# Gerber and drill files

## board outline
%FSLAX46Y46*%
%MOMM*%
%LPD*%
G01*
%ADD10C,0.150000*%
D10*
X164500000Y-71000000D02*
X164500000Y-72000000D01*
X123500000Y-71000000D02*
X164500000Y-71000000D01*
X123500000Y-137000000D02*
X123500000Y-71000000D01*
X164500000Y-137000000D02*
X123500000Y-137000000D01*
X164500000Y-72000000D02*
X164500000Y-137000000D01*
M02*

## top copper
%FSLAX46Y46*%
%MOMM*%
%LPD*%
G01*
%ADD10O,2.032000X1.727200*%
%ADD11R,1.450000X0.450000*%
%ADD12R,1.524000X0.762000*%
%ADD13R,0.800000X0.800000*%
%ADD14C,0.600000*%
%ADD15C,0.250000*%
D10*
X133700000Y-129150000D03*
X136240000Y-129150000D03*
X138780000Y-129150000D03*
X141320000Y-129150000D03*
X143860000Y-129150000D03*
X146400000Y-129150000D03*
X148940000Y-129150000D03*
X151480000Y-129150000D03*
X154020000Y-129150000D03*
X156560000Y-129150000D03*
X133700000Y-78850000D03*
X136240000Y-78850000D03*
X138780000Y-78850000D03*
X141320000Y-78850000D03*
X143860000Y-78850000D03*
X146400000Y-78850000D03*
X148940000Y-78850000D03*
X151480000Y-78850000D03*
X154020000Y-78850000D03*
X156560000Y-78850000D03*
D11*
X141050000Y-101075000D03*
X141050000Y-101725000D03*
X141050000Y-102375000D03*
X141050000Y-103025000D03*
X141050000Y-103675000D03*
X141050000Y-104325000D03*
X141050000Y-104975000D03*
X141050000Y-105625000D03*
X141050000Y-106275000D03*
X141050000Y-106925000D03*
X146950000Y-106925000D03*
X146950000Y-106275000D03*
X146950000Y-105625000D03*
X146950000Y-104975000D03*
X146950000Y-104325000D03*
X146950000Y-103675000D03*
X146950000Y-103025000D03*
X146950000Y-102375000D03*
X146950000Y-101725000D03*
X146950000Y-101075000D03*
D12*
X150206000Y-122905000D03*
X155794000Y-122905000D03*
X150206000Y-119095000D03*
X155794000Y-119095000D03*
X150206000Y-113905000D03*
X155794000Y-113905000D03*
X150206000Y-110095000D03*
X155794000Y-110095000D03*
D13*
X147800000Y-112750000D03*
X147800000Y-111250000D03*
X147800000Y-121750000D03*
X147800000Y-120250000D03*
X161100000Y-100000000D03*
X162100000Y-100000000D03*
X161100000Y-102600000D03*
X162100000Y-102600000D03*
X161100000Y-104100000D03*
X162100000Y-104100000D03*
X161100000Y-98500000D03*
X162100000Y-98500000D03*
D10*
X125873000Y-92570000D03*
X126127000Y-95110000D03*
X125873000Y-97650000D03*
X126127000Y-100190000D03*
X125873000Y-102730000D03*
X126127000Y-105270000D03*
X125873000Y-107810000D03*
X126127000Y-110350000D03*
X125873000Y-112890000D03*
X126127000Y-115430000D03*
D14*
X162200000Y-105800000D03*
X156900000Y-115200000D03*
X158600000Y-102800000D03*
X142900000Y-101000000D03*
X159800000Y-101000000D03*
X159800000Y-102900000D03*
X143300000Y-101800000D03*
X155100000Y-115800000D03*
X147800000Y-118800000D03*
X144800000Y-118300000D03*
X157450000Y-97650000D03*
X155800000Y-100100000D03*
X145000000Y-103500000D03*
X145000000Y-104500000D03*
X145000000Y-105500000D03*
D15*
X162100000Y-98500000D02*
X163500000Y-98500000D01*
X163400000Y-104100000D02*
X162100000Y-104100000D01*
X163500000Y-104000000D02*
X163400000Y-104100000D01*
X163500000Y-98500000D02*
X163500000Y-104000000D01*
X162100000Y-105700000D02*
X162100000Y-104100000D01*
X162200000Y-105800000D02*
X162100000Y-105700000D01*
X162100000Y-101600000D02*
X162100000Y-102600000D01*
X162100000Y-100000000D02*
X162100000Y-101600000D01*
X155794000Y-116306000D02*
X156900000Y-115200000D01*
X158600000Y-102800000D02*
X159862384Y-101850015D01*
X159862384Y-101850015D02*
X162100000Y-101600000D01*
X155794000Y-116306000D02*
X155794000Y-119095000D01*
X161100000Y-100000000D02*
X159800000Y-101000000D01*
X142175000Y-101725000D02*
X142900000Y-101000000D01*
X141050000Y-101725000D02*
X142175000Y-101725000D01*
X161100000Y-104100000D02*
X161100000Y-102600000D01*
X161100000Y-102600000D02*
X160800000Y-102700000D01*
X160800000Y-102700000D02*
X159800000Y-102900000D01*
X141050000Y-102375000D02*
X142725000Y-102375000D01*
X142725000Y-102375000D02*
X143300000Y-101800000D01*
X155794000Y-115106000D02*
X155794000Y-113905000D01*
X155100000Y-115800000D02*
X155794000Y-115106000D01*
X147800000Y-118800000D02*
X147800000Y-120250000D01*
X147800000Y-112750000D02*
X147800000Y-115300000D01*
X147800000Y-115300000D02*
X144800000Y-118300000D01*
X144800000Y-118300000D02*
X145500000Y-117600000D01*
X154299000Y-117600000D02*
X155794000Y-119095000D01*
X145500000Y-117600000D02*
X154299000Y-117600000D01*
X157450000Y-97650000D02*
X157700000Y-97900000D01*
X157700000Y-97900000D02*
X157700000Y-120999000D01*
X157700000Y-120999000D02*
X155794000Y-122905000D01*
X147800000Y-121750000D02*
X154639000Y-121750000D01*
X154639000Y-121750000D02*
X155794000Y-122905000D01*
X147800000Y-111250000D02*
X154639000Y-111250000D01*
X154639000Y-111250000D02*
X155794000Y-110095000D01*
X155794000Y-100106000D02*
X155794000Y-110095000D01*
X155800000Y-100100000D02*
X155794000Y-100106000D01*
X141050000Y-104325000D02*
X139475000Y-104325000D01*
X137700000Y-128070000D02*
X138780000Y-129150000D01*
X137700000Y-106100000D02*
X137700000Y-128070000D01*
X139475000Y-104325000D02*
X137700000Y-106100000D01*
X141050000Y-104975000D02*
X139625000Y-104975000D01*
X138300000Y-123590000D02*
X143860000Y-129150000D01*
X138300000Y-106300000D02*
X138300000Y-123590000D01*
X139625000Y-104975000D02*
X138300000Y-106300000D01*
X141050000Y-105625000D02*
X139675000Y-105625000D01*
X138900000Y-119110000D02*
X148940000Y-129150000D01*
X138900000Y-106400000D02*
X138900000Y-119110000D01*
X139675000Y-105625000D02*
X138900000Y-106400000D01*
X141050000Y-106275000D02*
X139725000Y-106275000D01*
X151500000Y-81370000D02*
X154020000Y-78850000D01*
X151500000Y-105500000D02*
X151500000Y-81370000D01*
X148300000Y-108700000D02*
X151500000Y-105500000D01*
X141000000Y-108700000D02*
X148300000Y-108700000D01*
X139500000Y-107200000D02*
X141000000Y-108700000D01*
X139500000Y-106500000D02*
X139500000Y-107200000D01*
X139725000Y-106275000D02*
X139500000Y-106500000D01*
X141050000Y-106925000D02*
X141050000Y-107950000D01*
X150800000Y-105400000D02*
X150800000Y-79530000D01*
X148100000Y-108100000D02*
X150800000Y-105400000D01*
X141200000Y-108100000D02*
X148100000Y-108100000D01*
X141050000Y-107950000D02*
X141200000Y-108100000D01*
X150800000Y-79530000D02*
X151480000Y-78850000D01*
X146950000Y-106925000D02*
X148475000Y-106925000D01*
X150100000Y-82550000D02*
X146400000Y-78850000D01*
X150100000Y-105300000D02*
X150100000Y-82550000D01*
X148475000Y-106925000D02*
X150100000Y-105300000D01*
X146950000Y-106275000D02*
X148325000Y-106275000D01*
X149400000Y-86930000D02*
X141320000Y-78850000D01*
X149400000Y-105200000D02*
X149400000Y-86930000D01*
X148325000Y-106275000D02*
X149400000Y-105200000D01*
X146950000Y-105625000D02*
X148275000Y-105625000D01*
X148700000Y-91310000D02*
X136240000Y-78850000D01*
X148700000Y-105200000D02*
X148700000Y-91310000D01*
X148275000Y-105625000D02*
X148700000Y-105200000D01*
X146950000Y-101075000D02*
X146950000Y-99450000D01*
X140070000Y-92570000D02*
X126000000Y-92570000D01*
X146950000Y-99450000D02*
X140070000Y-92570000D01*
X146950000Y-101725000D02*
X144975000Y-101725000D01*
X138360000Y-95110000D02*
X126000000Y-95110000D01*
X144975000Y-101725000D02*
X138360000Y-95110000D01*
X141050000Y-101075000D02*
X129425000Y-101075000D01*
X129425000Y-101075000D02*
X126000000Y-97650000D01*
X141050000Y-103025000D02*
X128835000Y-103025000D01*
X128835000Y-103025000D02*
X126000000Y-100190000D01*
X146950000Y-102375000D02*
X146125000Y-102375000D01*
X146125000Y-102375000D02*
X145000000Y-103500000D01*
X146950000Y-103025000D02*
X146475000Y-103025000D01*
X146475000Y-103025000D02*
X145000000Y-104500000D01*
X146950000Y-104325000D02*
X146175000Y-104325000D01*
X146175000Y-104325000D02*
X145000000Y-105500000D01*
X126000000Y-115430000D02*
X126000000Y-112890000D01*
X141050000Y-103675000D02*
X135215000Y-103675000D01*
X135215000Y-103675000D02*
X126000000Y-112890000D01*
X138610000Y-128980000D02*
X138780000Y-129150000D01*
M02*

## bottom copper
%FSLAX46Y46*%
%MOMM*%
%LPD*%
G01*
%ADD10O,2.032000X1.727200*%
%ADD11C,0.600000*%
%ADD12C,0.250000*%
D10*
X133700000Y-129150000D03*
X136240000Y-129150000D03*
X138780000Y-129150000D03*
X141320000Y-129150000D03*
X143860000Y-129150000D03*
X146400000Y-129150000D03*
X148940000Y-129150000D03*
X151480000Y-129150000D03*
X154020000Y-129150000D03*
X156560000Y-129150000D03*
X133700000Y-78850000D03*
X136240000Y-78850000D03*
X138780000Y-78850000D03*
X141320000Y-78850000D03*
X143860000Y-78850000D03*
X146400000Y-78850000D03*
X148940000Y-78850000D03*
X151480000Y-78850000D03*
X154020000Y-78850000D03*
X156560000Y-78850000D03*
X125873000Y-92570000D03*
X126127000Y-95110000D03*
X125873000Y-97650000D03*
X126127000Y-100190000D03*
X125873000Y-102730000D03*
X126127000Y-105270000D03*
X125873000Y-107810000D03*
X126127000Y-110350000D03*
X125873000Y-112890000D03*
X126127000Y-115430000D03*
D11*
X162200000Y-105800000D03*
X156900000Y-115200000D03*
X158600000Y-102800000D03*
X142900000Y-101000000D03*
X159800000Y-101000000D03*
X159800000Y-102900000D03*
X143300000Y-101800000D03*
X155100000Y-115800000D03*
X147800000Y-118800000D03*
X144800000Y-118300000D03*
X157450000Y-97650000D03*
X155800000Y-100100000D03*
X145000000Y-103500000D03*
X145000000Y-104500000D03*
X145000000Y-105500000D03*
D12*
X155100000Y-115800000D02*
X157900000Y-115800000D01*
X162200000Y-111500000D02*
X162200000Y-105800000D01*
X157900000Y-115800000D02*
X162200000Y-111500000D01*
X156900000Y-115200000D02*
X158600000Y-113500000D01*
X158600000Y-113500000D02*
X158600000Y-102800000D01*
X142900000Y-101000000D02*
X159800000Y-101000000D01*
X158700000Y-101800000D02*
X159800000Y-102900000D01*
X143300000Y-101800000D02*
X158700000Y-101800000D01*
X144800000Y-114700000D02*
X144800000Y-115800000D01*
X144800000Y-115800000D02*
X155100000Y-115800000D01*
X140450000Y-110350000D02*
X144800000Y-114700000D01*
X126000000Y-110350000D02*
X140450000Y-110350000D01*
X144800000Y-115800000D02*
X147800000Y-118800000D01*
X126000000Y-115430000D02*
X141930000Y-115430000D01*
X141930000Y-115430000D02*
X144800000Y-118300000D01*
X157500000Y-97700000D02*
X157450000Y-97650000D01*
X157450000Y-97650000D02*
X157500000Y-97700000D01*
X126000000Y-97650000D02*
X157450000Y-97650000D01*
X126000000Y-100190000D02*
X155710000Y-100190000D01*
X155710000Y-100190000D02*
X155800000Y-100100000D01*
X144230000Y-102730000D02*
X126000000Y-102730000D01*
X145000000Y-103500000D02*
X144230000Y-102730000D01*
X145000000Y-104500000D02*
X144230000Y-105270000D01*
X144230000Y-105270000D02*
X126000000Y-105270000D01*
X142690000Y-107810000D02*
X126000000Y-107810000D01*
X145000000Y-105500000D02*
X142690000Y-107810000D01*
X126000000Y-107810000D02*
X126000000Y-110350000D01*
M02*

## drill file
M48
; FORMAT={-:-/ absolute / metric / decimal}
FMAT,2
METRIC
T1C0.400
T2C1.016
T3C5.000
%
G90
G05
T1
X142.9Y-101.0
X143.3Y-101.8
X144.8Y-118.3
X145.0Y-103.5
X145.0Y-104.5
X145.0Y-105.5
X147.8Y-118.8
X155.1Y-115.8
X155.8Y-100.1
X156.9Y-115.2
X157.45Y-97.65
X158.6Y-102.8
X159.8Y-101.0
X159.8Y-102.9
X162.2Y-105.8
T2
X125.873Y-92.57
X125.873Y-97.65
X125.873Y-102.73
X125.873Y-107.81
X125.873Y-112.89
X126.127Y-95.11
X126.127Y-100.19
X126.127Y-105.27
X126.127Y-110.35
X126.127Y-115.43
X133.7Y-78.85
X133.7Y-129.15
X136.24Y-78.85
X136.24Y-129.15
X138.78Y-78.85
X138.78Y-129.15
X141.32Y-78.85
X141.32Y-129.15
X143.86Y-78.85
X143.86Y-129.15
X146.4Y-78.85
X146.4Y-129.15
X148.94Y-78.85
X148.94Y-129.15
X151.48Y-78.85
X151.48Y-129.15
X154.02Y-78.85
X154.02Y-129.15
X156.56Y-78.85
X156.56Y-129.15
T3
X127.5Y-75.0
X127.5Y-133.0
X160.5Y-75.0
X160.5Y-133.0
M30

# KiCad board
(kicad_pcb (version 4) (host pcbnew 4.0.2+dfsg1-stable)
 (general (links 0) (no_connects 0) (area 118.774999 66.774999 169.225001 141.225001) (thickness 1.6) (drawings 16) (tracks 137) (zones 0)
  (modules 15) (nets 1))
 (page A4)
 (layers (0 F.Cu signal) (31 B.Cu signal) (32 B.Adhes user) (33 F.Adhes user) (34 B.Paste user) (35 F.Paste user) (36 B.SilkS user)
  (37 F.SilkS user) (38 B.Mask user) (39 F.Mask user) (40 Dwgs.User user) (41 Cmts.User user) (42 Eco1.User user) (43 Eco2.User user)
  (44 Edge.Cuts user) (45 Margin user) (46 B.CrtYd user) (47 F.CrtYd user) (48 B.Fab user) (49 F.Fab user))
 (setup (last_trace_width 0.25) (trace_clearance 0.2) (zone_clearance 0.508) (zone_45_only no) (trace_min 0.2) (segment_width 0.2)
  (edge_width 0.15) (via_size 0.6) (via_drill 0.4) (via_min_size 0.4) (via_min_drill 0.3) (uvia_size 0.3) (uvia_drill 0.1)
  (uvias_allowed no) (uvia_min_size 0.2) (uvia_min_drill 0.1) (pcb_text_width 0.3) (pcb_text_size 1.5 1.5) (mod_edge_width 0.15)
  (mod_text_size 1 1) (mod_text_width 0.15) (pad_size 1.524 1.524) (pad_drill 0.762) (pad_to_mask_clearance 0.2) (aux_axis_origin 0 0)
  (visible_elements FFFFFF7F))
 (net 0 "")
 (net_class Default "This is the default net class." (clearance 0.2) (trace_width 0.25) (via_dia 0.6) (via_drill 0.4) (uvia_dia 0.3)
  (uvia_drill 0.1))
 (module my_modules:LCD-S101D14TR (layer B.Cu) (at 144 104 180)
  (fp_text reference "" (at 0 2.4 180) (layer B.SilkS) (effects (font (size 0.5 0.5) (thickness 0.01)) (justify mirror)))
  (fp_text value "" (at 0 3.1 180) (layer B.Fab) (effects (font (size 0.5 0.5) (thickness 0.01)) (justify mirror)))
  (pad 10 thru_hole oval (at 10.3 -25.15 180) (size 2.032 1.7272) (drill 1.016) (layers *.Cu *.Mask B.SilkS))
  (pad 9 thru_hole oval (at 7.76 -25.15 180) (size 2.032 1.7272) (drill 1.016) (layers *.Cu *.Mask B.SilkS))
  (pad 8 thru_hole oval (at 5.22 -25.15 180) (size 2.032 1.7272) (drill 1.016) (layers *.Cu *.Mask B.SilkS))
  (pad 7 thru_hole oval (at 2.68 -25.15 180) (size 2.032 1.7272) (drill 1.016) (layers *.Cu *.Mask B.SilkS))
  (pad 6 thru_hole oval (at 0.14 -25.15 180) (size 2.032 1.7272) (drill 1.016) (layers *.Cu *.Mask B.SilkS))
  (pad 5 thru_hole oval (at -2.4 -25.15 180) (size 2.032 1.7272) (drill 1.016) (layers *.Cu *.Mask B.SilkS))
  (pad 4 thru_hole oval (at -4.94 -25.15 180) (size 2.032 1.7272) (drill 1.016) (layers *.Cu *.Mask B.SilkS))
  (pad 3 thru_hole oval (at -7.48 -25.15 180) (size 2.032 1.7272) (drill 1.016) (layers *.Cu *.Mask B.SilkS))
  (pad 2 thru_hole oval (at -10.02 -25.15 180) (size 2.032 1.7272) (drill 1.016) (layers *.Cu *.Mask B.SilkS))
  (pad 1 thru_hole oval (at -12.56 -25.15 180) (size 2.032 1.7272) (drill 1.016) (layers *.Cu *.Mask B.SilkS))
  (pad 11 thru_hole oval (at 10.3 25.15 180) (size 2.032 1.7272) (drill 1.016) (layers *.Cu *.Mask B.SilkS))
  (pad 12 thru_hole oval (at 7.76 25.15 180) (size 2.032 1.7272) (drill 1.016) (layers *.Cu *.Mask B.SilkS))
  (pad 13 thru_hole oval (at 5.22 25.15 180) (size 2.032 1.7272) (drill 1.016) (layers *.Cu *.Mask B.SilkS))
  (pad 14 thru_hole oval (at 2.68 25.15 180) (size 2.032 1.7272) (drill 1.016) (layers *.Cu *.Mask B.SilkS))
  (pad 15 thru_hole oval (at 0.14 25.15 180) (size 2.032 1.7272) (drill 1.016) (layers *.Cu *.Mask B.SilkS))
  (pad 16 thru_hole oval (at -2.4 25.15 180) (size 2.032 1.7272) (drill 1.016) (layers *.Cu *.Mask B.SilkS))
  (pad 17 thru_hole oval (at -4.94 25.15 180) (size 2.032 1.7272) (drill 1.016) (layers *.Cu *.Mask B.SilkS))
  (pad 18 thru_hole oval (at -7.48 25.15 180) (size 2.032 1.7272) (drill 1.016) (layers *.Cu *.Mask B.SilkS))
  (pad 19 thru_hole oval (at -10.02 25.15 180) (size 2.032 1.7272) (drill 1.016) (layers *.Cu *.Mask B.SilkS))
  (pad 20 thru_hole oval (at -12.56 25.15 180) (size 2.032 1.7272) (drill 1.016) (layers *.Cu *.Mask B.SilkS)))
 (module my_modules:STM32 (layer F.Cu) (at 144 104)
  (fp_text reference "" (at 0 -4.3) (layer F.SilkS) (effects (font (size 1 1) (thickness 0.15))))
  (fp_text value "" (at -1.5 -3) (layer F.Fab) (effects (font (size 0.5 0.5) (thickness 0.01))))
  (pad BOOT smd rect (at -2.95 -2.925) (size 1.45 0.45) (layers F.Cu F.Paste F.Mask))
  (pad 2 smd rect (at -2.95 -2.275) (size 1.45 0.45) (layers F.Cu F.Paste F.Mask))
  (pad 3 smd rect (at -2.95 -1.625) (size 1.45 0.45) (layers F.Cu F.Paste F.Mask))
  (pad NRST smd rect (at -2.95 -0.975) (size 1.45 0.45) (layers F.Cu F.Paste F.Mask))
  (pad VCC smd rect (at -2.95 -0.325) (size 1.45 0.45) (layers F.Cu F.Paste F.Mask))
  (pad PA0 smd rect (at -2.95 0.325) (size 1.45 0.45) (layers F.Cu F.Paste F.Mask))
  (pad PA1 smd rect (at -2.95 0.975) (size 1.45 0.45) (layers F.Cu F.Paste F.Mask))
  (pad PA2 smd rect (at -2.95 1.625) (size 1.45 0.45) (layers F.Cu F.Paste F.Mask))
  (pad PA3 smd rect (at -2.95 2.275) (size 1.45 0.45) (layers F.Cu F.Paste F.Mask))
  (pad PA4 smd rect (at -2.95 2.925) (size 1.45 0.45) (layers F.Cu F.Paste F.Mask))
  (pad PA5 smd rect (at 2.95 2.925) (size 1.45 0.45) (layers F.Cu F.Paste F.Mask))
  (pad PA6 smd rect (at 2.95 2.275) (size 1.45 0.45) (layers F.Cu F.Paste F.Mask))
  (pad PA7 smd rect (at 2.95 1.625) (size 1.45 0.45) (layers F.Cu F.Paste F.Mask))
  (pad PB1 smd rect (at 2.95 0.975) (size 1.45 0.45) (layers F.Cu F.Paste F.Mask))
  (pad GND smd rect (at 2.95 0.325) (size 1.45 0.45) (layers F.Cu F.Paste F.Mask))
  (pad VCC smd rect (at 2.95 -0.325) (size 1.45 0.45) (layers F.Cu F.Paste F.Mask))
  (pad TX smd rect (at 2.95 -0.975) (size 1.45 0.45) (layers F.Cu F.Paste F.Mask))
  (pad RX smd rect (at 2.95 -1.625) (size 1.45 0.45) (layers F.Cu F.Paste F.Mask))
  (pad DIO smd rect (at 2.95 -2.275) (size 1.45 0.45) (layers F.Cu F.Paste F.Mask))
  (pad CLK smd rect (at 2.95 -2.925) (size 1.45 0.45) (layers F.Cu F.Paste F.Mask)))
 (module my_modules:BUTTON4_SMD (layer F.Cu) (at 153 121)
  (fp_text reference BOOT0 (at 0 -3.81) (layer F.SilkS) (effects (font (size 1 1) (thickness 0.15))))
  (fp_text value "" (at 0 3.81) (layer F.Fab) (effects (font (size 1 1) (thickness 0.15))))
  (pad 1 smd rect (at -2.794 1.905) (size 1.524 0.762) (layers F.Cu F.Paste F.Mask))
  (pad 2 smd rect (at 2.794 1.905) (size 1.524 0.762) (layers F.Cu F.Paste F.Mask))
  (pad 3 smd rect (at -2.794 -1.905) (size 1.524 0.762) (layers F.Cu F.Paste F.Mask))
  (pad 4 smd rect (at 2.794 -1.905) (size 1.524 0.762) (layers F.Cu F.Paste F.Mask)))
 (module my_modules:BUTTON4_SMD (layer F.Cu) (at 153 112)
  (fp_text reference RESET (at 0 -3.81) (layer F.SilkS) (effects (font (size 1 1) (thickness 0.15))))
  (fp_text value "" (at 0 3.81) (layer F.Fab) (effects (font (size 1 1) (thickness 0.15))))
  (pad 1 smd rect (at -2.794 1.905) (size 1.524 0.762) (layers F.Cu F.Paste F.Mask))
  (pad 2 smd rect (at 2.794 1.905) (size 1.524 0.762) (layers F.Cu F.Paste F.Mask))
  (pad 3 smd rect (at -2.794 -1.905) (size 1.524 0.762) (layers F.Cu F.Paste F.Mask))
  (pad 4 smd rect (at 2.794 -1.905) (size 1.524 0.762) (layers F.Cu F.Paste F.Mask)))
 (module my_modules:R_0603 (layer F.Cu) (at 147.8 112 90)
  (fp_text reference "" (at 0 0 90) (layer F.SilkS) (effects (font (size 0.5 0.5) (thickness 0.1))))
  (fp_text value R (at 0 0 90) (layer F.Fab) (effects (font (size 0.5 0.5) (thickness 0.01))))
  (pad 1 smd rect (at -0.75 0 90) (size 0.8 0.8) (layers F.Cu F.Paste F.Mask))
  (pad 2 smd rect (at 0.75 0 90) (size 0.8 0.8) (layers F.Cu F.Paste F.Mask)))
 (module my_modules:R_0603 (layer F.Cu) (at 147.8 121 90)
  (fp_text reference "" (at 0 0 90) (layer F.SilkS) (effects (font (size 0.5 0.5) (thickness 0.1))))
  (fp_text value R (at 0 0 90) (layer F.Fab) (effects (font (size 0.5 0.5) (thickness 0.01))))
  (pad 1 smd rect (at -0.75 0 90) (size 0.8 0.8) (layers F.Cu F.Paste F.Mask))
  (pad 2 smd rect (at 0.75 0 90) (size 0.8 0.8) (layers F.Cu F.Paste F.Mask)))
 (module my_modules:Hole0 (layer F.Cu) (at 160.5 133)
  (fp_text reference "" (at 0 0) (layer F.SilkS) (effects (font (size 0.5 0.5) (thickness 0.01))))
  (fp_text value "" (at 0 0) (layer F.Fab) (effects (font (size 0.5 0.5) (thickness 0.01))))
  (pad "" np_thru_hole circle (at 0 0) (size 5 5) (drill 5) (layers *.Cu *.Mask F.SilkS)))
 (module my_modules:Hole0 (layer F.Cu) (at 127.5 133)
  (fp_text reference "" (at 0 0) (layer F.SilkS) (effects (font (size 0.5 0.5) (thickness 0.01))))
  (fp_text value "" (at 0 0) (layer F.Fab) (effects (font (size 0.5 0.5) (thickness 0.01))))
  (pad "" np_thru_hole circle (at 0 0) (size 5 5) (drill 5) (layers *.Cu *.Mask F.SilkS)))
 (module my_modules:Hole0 (layer F.Cu) (at 160.5 75)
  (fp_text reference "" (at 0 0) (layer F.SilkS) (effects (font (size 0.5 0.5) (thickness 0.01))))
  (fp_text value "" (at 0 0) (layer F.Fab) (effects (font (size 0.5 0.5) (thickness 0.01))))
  (pad "" np_thru_hole circle (at 0 0) (size 5 5) (drill 5) (layers *.Cu *.Mask F.SilkS)))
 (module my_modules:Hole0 (layer F.Cu) (at 127.5 75)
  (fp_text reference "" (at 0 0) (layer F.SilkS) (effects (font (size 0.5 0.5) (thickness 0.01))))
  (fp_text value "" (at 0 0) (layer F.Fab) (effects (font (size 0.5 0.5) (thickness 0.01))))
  (pad "" np_thru_hole circle (at 0 0) (size 5 5) (drill 5) (layers *.Cu *.Mask F.SilkS)))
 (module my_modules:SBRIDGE (layer F.Cu) (at 161.6 100)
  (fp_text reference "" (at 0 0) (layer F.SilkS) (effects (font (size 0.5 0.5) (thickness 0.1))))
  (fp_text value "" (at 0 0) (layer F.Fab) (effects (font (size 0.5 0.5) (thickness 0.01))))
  (pad 1 smd rect (at -0.5 0) (size 0.8 0.8) (layers F.Cu F.Paste F.Mask))
  (pad 2 smd rect (at 0.5 0) (size 0.8 0.8) (layers F.Cu F.Paste F.Mask)))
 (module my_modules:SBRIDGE (layer F.Cu) (at 161.6 102.6)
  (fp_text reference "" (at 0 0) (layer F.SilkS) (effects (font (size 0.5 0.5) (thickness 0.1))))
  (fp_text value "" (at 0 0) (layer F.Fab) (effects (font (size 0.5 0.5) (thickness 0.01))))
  (pad 1 smd rect (at -0.5 0) (size 0.8 0.8) (layers F.Cu F.Paste F.Mask))
  (pad 2 smd rect (at 0.5 0) (size 0.8 0.8) (layers F.Cu F.Paste F.Mask)))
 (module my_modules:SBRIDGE (layer F.Cu) (at 161.6 104.1)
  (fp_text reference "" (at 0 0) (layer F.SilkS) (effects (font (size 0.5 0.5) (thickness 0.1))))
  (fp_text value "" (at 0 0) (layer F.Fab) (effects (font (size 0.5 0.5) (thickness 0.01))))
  (pad 1 smd rect (at -0.5 0) (size 0.8 0.8) (layers F.Cu F.Paste F.Mask))
  (pad 2 smd rect (at 0.5 0) (size 0.8 0.8) (layers F.Cu F.Paste F.Mask)))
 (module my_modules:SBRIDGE (layer F.Cu) (at 161.6 98.5)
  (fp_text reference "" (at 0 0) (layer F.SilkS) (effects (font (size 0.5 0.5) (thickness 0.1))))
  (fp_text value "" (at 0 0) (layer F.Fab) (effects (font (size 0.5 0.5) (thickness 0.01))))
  (pad 1 smd rect (at -0.5 0) (size 0.8 0.8) (layers F.Cu F.Paste F.Mask))
  (pad 2 smd rect (at 0.5 0) (size 0.8 0.8) (layers F.Cu F.Paste F.Mask)))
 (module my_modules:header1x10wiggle (layer F.Cu) (at 126 104)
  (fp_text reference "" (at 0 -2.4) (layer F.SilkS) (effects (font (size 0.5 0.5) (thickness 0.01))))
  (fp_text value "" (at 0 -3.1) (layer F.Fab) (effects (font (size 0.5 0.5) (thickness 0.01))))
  (pad 2 thru_hole oval (at -0.127 -11.43) (size 2.032 1.7272) (drill 1.016) (layers *.Cu *.Mask F.SilkS))
  (pad 3 thru_hole oval (at 0.127 -8.89) (size 2.032 1.7272) (drill 1.016) (layers *.Cu *.Mask F.SilkS))
  (pad 4 thru_hole oval (at -0.127 -6.35) (size 2.032 1.7272) (drill 1.016) (layers *.Cu *.Mask F.SilkS))
  (pad 5 thru_hole oval (at 0.127 -3.81) (size 2.032 1.7272) (drill 1.016) (layers *.Cu *.Mask F.SilkS))
  (pad 6 thru_hole oval (at -0.127 -1.27) (size 2.032 1.7272) (drill 1.016) (layers *.Cu *.Mask F.SilkS))
  (pad 7 thru_hole oval (at 0.127 1.27) (size 2.032 1.7272) (drill 1.016) (layers *.Cu *.Mask F.SilkS))
  (pad 8 thru_hole oval (at -0.127 3.81) (size 2.032 1.7272) (drill 1.016) (layers *.Cu *.Mask F.SilkS))
  (pad 9 thru_hole oval (at 0.127 6.35) (size 2.032 1.7272) (drill 1.016) (layers *.Cu *.Mask F.SilkS))
  (pad 10 thru_hole oval (at -0.127 8.89) (size 2.032 1.7272) (drill 1.016) (layers *.Cu *.Mask F.SilkS))
  (pad 11 thru_hole oval (at 0.127 11.43) (size 2.032 1.7272) (drill 1.016) (layers *.Cu *.Mask F.SilkS)))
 (gr_line (start 164.5 71) (end 164.5 72) (angle 90) (layer Edge.Cuts) (width 0.15))
 (gr_line (start 123.5 71) (end 164.5 71) (angle 90) (layer Edge.Cuts) (width 0.15))
 (gr_line (start 123.5 137) (end 123.5 71) (angle 90) (layer Edge.Cuts) (width 0.15))
 (gr_line (start 164.5 137) (end 123.5 137) (angle 90) (layer Edge.Cuts) (width 0.15))
 (gr_line (start 164.5 72) (end 164.5 137) (angle 90) (layer Edge.Cuts) (width 0.15))
 (segment (start 162.1 98.5) (end 163.5 98.5) (width 0.25) (layer F.Cu) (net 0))
 (segment (start 163.4 104.1) (end 162.1 104.1) (width 0.25) (layer F.Cu) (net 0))
 (segment (start 163.5 104) (end 163.4 104.1) (width 0.25) (layer F.Cu) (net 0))
 (segment (start 163.5 98.5) (end 163.5 104) (width 0.25) (layer F.Cu) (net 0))
 (segment (start 155.1 115.8) (end 157.9 115.8) (width 0.25) (layer B.Cu) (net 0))
 (segment (start 162.1 105.7) (end 162.1 104.1) (width 0.25) (layer F.Cu) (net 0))
 (segment (start 162.2 105.8) (end 162.1 105.7) (width 0.25) (layer F.Cu) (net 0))
 (via (at 162.2 105.8) (size 0.6) (drill 0.4) (layers F.Cu B.Cu) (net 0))
 (segment (start 162.2 111.5) (end 162.2 105.8) (width 0.25) (layer B.Cu) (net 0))
 (segment (start 157.9 115.8) (end 162.2 111.5) (width 0.25) (layer B.Cu) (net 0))
 (segment (start 162.1 101.6) (end 162.1 102.6) (width 0.25) (layer F.Cu) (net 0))
 (segment (start 162.1 100) (end 162.1 101.6) (width 0.25) (layer F.Cu) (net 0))
 (segment (start 155.794 116.306) (end 156.9 115.2) (width 0.25) (layer F.Cu) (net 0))
 (via (at 156.9 115.2) (size 0.6) (drill 0.4) (layers F.Cu B.Cu) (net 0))
 (segment (start 156.9 115.2) (end 158.6 113.5) (width 0.25) (layer B.Cu) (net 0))
 (segment (start 158.6 113.5) (end 158.6 102.8) (width 0.25) (layer B.Cu) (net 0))
 (via (at 158.6 102.8) (size 0.6) (drill 0.4) (layers F.Cu B.Cu) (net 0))
 (segment (start 158.6 102.8) (end 159.862384 101.850015) (width 0.25) (layer F.Cu) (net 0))
 (segment (start 159.862384 101.850015) (end 162.1 101.6) (width 0.25) (layer F.Cu) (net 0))
 (segment (start 155.794 116.306) (end 155.794 119.095) (width 0.25) (layer F.Cu) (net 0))
 (segment (start 161.1 100) (end 159.8 101) (width 0.25) (layer F.Cu) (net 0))
 (segment (start 142.175 101.725) (end 142.9 101) (width 0.25) (layer F.Cu) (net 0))
 (via (at 142.9 101) (size 0.6) (drill 0.4) (layers F.Cu B.Cu) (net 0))
 (segment (start 142.9 101) (end 159.8 101) (width 0.25) (layer B.Cu) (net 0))
 (via (at 159.8 101) (size 0.6) (drill 0.4) (layers F.Cu B.Cu) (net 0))
 (segment (start 141.05 101.725) (end 142.175 101.725) (width 0.25) (layer F.Cu) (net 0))
 (segment (start 161.1 104.1) (end 161.1 102.6) (width 0.25) (layer F.Cu) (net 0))
 (segment (start 161.1 102.6) (end 160.8 102.7) (width 0.25) (layer F.Cu) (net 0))
 (segment (start 160.8 102.7) (end 159.8 102.9) (width 0.25) (layer F.Cu) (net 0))
 (segment (start 141.05 102.375) (end 142.725 102.375) (width 0.25) (layer F.Cu) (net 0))
 (via (at 159.8 102.9) (size 0.6) (drill 0.4) (layers F.Cu B.Cu) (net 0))
 (segment (start 158.7 101.8) (end 159.8 102.9) (width 0.25) (layer B.Cu) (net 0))
 (segment (start 143.3 101.8) (end 158.7 101.8) (width 0.25) (layer B.Cu) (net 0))
 (via (at 143.3 101.8) (size 0.6) (drill 0.4) (layers F.Cu B.Cu) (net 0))
 (segment (start 142.725 102.375) (end 143.3 101.8) (width 0.25) (layer F.Cu) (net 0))
 (segment (start 144.8 114.7) (end 144.8 115.8) (width 0.25) (layer B.Cu) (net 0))
 (segment (start 144.8 115.8) (end 155.1 115.8) (width 0.25) (layer B.Cu) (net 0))
 (segment (start 155.794 115.106) (end 155.794 113.905) (width 0.25) (layer F.Cu) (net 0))
 (segment (start 155.1 115.8) (end 155.794 115.106) (width 0.25) (layer F.Cu) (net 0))
 (via (at 155.1 115.8) (size 0.6) (drill 0.4) (layers F.Cu B.Cu) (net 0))
 (segment (start 140.45 110.35) (end 144.8 114.7) (width 0.25) (layer B.Cu) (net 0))
 (segment (start 126 110.35) (end 140.45 110.35) (width 0.25) (layer B.Cu) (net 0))
 (segment (start 147.8 118.8) (end 147.8 120.25) (width 0.25) (layer F.Cu) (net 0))
 (via (at 147.8 118.8) (size 0.6) (drill 0.4) (layers F.Cu B.Cu) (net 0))
 (segment (start 144.8 115.8) (end 147.8 118.8) (width 0.25) (layer B.Cu) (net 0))
 (segment (start 147.8 112.75) (end 147.8 115.3) (width 0.25) (layer F.Cu) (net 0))
 (segment (start 147.8 115.3) (end 144.8 118.3) (width 0.25) (layer F.Cu) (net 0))
 (segment (start 144.8 118.3) (end 145.5 117.6) (width 0.25) (layer F.Cu) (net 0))
 (segment (start 126 115.43) (end 141.93 115.43) (width 0.25) (layer B.Cu) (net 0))
 (via (at 144.8 118.3) (size 0.6) (drill 0.4) (layers F.Cu B.Cu) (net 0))
 (segment (start 141.93 115.43) (end 144.8 118.3) (width 0.25) (layer B.Cu) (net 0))
 (segment (start 154.299 117.6) (end 155.794 119.095) (width 0.25) (layer F.Cu) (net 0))
 (segment (start 145.5 117.6) (end 154.299 117.6) (width 0.25) (layer F.Cu) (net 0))
 (segment (start 157.5 97.7) (end 157.45 97.65) (width 0.25) (layer B.Cu) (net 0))
 (segment (start 157.45 97.65) (end 157.5 97.7) (width 0.25) (layer B.Cu) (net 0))
 (via (at 157.45 97.65) (size 0.6) (drill 0.4) (layers F.Cu B.Cu) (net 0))
 (segment (start 157.45 97.65) (end 157.7 97.9) (width 0.25) (layer F.Cu) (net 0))
 (segment (start 157.7 97.9) (end 157.7 120.999) (width 0.25) (layer F.Cu) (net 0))
 (segment (start 157.7 120.999) (end 155.794 122.905) (width 0.25) (layer F.Cu) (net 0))
 (segment (start 126 97.65) (end 157.45 97.65) (width 0.25) (layer B.Cu) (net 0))
 (segment (start 147.8 121.75) (end 154.639 121.75) (width 0.25) (layer F.Cu) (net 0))
 (segment (start 154.639 121.75) (end 155.794 122.905) (width 0.25) (layer F.Cu) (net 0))
 (segment (start 147.8 111.25) (end 154.639 111.25) (width 0.25) (layer F.Cu) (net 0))
 (segment (start 154.639 111.25) (end 155.794 110.095) (width 0.25) (layer F.Cu) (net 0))
 (segment (start 126 100.19) (end 155.71 100.19) (width 0.25) (layer B.Cu) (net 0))
 (segment (start 155.794 100.106) (end 155.794 110.095) (width 0.25) (layer F.Cu) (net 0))
 (segment (start 155.8 100.1) (end 155.794 100.106) (width 0.25) (layer F.Cu) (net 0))
 (via (at 155.8 100.1) (size 0.6) (drill 0.4) (layers F.Cu B.Cu) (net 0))
 (segment (start 155.71 100.19) (end 155.8 100.1) (width 0.25) (layer B.Cu) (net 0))
 (segment (start 141.05 104.325) (end 139.475 104.325) (width 0.25) (layer F.Cu) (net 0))
 (segment (start 137.7 128.07) (end 138.78 129.15) (width 0.25) (layer F.Cu) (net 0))
 (segment (start 137.7 106.1) (end 137.7 128.07) (width 0.25) (layer F.Cu) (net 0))
 (segment (start 139.475 104.325) (end 137.7 106.1) (width 0.25) (layer F.Cu) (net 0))
 (segment (start 141.05 104.975) (end 139.625 104.975) (width 0.25) (layer F.Cu) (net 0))
 (segment (start 138.3 123.59) (end 143.86 129.15) (width 0.25) (layer F.Cu) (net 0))
 (segment (start 138.3 106.3) (end 138.3 123.59) (width 0.25) (layer F.Cu) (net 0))
 (segment (start 139.625 104.975) (end 138.3 106.3) (width 0.25) (layer F.Cu) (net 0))
 (segment (start 141.05 105.625) (end 139.675 105.625) (width 0.25) (layer F.Cu) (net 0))
 (segment (start 138.9 119.11) (end 148.94 129.15) (width 0.25) (layer F.Cu) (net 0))
 (segment (start 138.9 106.4) (end 138.9 119.11) (width 0.25) (layer F.Cu) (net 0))
 (segment (start 139.675 105.625) (end 138.9 106.4) (width 0.25) (layer F.Cu) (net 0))
 (segment (start 141.05 106.275) (end 139.725 106.275) (width 0.25) (layer F.Cu) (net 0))
 (segment (start 151.5 81.37) (end 154.02 78.85) (width 0.25) (layer F.Cu) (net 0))
 (segment (start 151.5 105.5) (end 151.5 81.37) (width 0.25) (layer F.Cu) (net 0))
 (segment (start 148.3 108.7) (end 151.5 105.5) (width 0.25) (layer F.Cu) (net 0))
 (segment (start 141 108.7) (end 148.3 108.7) (width 0.25) (layer F.Cu) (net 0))
 (segment (start 139.5 107.2) (end 141 108.7) (width 0.25) (layer F.Cu) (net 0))
 (segment (start 139.5 106.5) (end 139.5 107.2) (width 0.25) (layer F.Cu) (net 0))
 (segment (start 139.725 106.275) (end 139.5 106.5) (width 0.25) (layer F.Cu) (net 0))
 (segment (start 141.05 106.925) (end 141.05 107.95) (width 0.25) (layer F.Cu) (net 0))
 (segment (start 150.8 105.4) (end 150.8 79.53) (width 0.25) (layer F.Cu) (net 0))
 (segment (start 148.1 108.1) (end 150.8 105.4) (width 0.25) (layer F.Cu) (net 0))
 (segment (start 141.2 108.1) (end 148.1 108.1) (width 0.25) (layer F.Cu) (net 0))
 (segment (start 141.05 107.95) (end 141.2 108.1) (width 0.25) (layer F.Cu) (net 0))
 (segment (start 150.8 79.53) (end 151.48 78.85) (width 0.25) (layer F.Cu) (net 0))
 (segment (start 146.95 106.925) (end 148.475 106.925) (width 0.25) (layer F.Cu) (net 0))
 (segment (start 150.1 82.55) (end 146.4 78.85) (width 0.25) (layer F.Cu) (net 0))
 (segment (start 150.1 105.3) (end 150.1 82.55) (width 0.25) (layer F.Cu) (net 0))
 (segment (start 148.475 106.925) (end 150.1 105.3) (width 0.25) (layer F.Cu) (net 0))
 (segment (start 146.95 106.275) (end 148.325 106.275) (width 0.25) (layer F.Cu) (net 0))
 (segment (start 149.4 86.93) (end 141.32 78.85) (width 0.25) (layer F.Cu) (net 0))
 (segment (start 149.4 105.2) (end 149.4 86.93) (width 0.25) (layer F.Cu) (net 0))
 (segment (start 148.325 106.275) (end 149.4 105.2) (width 0.25) (layer F.Cu) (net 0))
 (segment (start 146.95 105.625) (end 148.275 105.625) (width 0.25) (layer F.Cu) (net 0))
 (segment (start 148.7 91.31) (end 136.24 78.85) (width 0.25) (layer F.Cu) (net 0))
 (segment (start 148.7 105.2) (end 148.7 91.31) (width 0.25) (layer F.Cu) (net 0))
 (segment (start 148.275 105.625) (end 148.7 105.2) (width 0.25) (layer F.Cu) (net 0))
 (segment (start 146.95 101.075) (end 146.95 99.45) (width 0.25) (layer F.Cu) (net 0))
 (segment (start 140.07 92.57) (end 126 92.57) (width 0.25) (layer F.Cu) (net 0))
 (segment (start 146.95 99.45) (end 140.07 92.57) (width 0.25) (layer F.Cu) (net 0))
 (segment (start 146.95 101.725) (end 144.975 101.725) (width 0.25) (layer F.Cu) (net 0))
 (segment (start 138.36 95.11) (end 126 95.11) (width 0.25) (layer F.Cu) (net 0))
 (segment (start 144.975 101.725) (end 138.36 95.11) (width 0.25) (layer F.Cu) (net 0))
 (segment (start 141.05 101.075) (end 129.425 101.075) (width 0.25) (layer F.Cu) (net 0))
 (segment (start 129.425 101.075) (end 126 97.65) (width 0.25) (layer F.Cu) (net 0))
 (segment (start 141.05 103.025) (end 128.835 103.025) (width 0.25) (layer F.Cu) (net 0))
 (segment (start 128.835 103.025) (end 126 100.19) (width 0.25) (layer F.Cu) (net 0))
 (segment (start 146.95 102.375) (end 146.125 102.375) (width 0.25) (layer F.Cu) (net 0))
 (segment (start 144.23 102.73) (end 126 102.73) (width 0.25) (layer B.Cu) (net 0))
 (segment (start 145 103.5) (end 144.23 102.73) (width 0.25) (layer B.Cu) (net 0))
 (via (at 145 103.5) (size 0.6) (drill 0.4) (layers F.Cu B.Cu) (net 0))
 (segment (start 146.125 102.375) (end 145 103.5) (width 0.25) (layer F.Cu) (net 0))
 (segment (start 146.95 103.025) (end 146.475 103.025) (width 0.25) (layer F.Cu) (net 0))
 (segment (start 146.475 103.025) (end 145 104.5) (width 0.25) (layer F.Cu) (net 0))
 (via (at 145 104.5) (size 0.6) (drill 0.4) (layers F.Cu B.Cu) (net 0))
 (segment (start 145 104.5) (end 144.23 105.27) (width 0.25) (layer B.Cu) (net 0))
 (segment (start 144.23 105.27) (end 126 105.27) (width 0.25) (layer B.Cu) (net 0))
 (segment (start 146.95 104.325) (end 146.175 104.325) (width 0.25) (layer F.Cu) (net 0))
 (segment (start 142.69 107.81) (end 126 107.81) (width 0.25) (layer B.Cu) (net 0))
 (segment (start 145 105.5) (end 142.69 107.81) (width 0.25) (layer B.Cu) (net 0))
 (via (at 145 105.5) (size 0.6) (drill 0.4) (layers F.Cu B.Cu) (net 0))
 (segment (start 146.175 104.325) (end 145 105.5) (width 0.25) (layer F.Cu) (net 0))
 (segment (start 126 107.81) (end 126 110.35) (width 0.25) (layer B.Cu) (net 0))
 (segment (start 126 115.43) (end 126 112.89) (width 0.25) (layer F.Cu) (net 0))
 (segment (start 141.05 103.675) (end 135.215 103.675) (width 0.25) (layer F.Cu) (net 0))
 (segment (start 135.215 103.675) (end 126 112.89) (width 0.25) (layer F.Cu) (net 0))
 (segment (start 138.61 128.98) (end 138.78 129.15) (width 0.25) (layer F.Cu) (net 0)))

